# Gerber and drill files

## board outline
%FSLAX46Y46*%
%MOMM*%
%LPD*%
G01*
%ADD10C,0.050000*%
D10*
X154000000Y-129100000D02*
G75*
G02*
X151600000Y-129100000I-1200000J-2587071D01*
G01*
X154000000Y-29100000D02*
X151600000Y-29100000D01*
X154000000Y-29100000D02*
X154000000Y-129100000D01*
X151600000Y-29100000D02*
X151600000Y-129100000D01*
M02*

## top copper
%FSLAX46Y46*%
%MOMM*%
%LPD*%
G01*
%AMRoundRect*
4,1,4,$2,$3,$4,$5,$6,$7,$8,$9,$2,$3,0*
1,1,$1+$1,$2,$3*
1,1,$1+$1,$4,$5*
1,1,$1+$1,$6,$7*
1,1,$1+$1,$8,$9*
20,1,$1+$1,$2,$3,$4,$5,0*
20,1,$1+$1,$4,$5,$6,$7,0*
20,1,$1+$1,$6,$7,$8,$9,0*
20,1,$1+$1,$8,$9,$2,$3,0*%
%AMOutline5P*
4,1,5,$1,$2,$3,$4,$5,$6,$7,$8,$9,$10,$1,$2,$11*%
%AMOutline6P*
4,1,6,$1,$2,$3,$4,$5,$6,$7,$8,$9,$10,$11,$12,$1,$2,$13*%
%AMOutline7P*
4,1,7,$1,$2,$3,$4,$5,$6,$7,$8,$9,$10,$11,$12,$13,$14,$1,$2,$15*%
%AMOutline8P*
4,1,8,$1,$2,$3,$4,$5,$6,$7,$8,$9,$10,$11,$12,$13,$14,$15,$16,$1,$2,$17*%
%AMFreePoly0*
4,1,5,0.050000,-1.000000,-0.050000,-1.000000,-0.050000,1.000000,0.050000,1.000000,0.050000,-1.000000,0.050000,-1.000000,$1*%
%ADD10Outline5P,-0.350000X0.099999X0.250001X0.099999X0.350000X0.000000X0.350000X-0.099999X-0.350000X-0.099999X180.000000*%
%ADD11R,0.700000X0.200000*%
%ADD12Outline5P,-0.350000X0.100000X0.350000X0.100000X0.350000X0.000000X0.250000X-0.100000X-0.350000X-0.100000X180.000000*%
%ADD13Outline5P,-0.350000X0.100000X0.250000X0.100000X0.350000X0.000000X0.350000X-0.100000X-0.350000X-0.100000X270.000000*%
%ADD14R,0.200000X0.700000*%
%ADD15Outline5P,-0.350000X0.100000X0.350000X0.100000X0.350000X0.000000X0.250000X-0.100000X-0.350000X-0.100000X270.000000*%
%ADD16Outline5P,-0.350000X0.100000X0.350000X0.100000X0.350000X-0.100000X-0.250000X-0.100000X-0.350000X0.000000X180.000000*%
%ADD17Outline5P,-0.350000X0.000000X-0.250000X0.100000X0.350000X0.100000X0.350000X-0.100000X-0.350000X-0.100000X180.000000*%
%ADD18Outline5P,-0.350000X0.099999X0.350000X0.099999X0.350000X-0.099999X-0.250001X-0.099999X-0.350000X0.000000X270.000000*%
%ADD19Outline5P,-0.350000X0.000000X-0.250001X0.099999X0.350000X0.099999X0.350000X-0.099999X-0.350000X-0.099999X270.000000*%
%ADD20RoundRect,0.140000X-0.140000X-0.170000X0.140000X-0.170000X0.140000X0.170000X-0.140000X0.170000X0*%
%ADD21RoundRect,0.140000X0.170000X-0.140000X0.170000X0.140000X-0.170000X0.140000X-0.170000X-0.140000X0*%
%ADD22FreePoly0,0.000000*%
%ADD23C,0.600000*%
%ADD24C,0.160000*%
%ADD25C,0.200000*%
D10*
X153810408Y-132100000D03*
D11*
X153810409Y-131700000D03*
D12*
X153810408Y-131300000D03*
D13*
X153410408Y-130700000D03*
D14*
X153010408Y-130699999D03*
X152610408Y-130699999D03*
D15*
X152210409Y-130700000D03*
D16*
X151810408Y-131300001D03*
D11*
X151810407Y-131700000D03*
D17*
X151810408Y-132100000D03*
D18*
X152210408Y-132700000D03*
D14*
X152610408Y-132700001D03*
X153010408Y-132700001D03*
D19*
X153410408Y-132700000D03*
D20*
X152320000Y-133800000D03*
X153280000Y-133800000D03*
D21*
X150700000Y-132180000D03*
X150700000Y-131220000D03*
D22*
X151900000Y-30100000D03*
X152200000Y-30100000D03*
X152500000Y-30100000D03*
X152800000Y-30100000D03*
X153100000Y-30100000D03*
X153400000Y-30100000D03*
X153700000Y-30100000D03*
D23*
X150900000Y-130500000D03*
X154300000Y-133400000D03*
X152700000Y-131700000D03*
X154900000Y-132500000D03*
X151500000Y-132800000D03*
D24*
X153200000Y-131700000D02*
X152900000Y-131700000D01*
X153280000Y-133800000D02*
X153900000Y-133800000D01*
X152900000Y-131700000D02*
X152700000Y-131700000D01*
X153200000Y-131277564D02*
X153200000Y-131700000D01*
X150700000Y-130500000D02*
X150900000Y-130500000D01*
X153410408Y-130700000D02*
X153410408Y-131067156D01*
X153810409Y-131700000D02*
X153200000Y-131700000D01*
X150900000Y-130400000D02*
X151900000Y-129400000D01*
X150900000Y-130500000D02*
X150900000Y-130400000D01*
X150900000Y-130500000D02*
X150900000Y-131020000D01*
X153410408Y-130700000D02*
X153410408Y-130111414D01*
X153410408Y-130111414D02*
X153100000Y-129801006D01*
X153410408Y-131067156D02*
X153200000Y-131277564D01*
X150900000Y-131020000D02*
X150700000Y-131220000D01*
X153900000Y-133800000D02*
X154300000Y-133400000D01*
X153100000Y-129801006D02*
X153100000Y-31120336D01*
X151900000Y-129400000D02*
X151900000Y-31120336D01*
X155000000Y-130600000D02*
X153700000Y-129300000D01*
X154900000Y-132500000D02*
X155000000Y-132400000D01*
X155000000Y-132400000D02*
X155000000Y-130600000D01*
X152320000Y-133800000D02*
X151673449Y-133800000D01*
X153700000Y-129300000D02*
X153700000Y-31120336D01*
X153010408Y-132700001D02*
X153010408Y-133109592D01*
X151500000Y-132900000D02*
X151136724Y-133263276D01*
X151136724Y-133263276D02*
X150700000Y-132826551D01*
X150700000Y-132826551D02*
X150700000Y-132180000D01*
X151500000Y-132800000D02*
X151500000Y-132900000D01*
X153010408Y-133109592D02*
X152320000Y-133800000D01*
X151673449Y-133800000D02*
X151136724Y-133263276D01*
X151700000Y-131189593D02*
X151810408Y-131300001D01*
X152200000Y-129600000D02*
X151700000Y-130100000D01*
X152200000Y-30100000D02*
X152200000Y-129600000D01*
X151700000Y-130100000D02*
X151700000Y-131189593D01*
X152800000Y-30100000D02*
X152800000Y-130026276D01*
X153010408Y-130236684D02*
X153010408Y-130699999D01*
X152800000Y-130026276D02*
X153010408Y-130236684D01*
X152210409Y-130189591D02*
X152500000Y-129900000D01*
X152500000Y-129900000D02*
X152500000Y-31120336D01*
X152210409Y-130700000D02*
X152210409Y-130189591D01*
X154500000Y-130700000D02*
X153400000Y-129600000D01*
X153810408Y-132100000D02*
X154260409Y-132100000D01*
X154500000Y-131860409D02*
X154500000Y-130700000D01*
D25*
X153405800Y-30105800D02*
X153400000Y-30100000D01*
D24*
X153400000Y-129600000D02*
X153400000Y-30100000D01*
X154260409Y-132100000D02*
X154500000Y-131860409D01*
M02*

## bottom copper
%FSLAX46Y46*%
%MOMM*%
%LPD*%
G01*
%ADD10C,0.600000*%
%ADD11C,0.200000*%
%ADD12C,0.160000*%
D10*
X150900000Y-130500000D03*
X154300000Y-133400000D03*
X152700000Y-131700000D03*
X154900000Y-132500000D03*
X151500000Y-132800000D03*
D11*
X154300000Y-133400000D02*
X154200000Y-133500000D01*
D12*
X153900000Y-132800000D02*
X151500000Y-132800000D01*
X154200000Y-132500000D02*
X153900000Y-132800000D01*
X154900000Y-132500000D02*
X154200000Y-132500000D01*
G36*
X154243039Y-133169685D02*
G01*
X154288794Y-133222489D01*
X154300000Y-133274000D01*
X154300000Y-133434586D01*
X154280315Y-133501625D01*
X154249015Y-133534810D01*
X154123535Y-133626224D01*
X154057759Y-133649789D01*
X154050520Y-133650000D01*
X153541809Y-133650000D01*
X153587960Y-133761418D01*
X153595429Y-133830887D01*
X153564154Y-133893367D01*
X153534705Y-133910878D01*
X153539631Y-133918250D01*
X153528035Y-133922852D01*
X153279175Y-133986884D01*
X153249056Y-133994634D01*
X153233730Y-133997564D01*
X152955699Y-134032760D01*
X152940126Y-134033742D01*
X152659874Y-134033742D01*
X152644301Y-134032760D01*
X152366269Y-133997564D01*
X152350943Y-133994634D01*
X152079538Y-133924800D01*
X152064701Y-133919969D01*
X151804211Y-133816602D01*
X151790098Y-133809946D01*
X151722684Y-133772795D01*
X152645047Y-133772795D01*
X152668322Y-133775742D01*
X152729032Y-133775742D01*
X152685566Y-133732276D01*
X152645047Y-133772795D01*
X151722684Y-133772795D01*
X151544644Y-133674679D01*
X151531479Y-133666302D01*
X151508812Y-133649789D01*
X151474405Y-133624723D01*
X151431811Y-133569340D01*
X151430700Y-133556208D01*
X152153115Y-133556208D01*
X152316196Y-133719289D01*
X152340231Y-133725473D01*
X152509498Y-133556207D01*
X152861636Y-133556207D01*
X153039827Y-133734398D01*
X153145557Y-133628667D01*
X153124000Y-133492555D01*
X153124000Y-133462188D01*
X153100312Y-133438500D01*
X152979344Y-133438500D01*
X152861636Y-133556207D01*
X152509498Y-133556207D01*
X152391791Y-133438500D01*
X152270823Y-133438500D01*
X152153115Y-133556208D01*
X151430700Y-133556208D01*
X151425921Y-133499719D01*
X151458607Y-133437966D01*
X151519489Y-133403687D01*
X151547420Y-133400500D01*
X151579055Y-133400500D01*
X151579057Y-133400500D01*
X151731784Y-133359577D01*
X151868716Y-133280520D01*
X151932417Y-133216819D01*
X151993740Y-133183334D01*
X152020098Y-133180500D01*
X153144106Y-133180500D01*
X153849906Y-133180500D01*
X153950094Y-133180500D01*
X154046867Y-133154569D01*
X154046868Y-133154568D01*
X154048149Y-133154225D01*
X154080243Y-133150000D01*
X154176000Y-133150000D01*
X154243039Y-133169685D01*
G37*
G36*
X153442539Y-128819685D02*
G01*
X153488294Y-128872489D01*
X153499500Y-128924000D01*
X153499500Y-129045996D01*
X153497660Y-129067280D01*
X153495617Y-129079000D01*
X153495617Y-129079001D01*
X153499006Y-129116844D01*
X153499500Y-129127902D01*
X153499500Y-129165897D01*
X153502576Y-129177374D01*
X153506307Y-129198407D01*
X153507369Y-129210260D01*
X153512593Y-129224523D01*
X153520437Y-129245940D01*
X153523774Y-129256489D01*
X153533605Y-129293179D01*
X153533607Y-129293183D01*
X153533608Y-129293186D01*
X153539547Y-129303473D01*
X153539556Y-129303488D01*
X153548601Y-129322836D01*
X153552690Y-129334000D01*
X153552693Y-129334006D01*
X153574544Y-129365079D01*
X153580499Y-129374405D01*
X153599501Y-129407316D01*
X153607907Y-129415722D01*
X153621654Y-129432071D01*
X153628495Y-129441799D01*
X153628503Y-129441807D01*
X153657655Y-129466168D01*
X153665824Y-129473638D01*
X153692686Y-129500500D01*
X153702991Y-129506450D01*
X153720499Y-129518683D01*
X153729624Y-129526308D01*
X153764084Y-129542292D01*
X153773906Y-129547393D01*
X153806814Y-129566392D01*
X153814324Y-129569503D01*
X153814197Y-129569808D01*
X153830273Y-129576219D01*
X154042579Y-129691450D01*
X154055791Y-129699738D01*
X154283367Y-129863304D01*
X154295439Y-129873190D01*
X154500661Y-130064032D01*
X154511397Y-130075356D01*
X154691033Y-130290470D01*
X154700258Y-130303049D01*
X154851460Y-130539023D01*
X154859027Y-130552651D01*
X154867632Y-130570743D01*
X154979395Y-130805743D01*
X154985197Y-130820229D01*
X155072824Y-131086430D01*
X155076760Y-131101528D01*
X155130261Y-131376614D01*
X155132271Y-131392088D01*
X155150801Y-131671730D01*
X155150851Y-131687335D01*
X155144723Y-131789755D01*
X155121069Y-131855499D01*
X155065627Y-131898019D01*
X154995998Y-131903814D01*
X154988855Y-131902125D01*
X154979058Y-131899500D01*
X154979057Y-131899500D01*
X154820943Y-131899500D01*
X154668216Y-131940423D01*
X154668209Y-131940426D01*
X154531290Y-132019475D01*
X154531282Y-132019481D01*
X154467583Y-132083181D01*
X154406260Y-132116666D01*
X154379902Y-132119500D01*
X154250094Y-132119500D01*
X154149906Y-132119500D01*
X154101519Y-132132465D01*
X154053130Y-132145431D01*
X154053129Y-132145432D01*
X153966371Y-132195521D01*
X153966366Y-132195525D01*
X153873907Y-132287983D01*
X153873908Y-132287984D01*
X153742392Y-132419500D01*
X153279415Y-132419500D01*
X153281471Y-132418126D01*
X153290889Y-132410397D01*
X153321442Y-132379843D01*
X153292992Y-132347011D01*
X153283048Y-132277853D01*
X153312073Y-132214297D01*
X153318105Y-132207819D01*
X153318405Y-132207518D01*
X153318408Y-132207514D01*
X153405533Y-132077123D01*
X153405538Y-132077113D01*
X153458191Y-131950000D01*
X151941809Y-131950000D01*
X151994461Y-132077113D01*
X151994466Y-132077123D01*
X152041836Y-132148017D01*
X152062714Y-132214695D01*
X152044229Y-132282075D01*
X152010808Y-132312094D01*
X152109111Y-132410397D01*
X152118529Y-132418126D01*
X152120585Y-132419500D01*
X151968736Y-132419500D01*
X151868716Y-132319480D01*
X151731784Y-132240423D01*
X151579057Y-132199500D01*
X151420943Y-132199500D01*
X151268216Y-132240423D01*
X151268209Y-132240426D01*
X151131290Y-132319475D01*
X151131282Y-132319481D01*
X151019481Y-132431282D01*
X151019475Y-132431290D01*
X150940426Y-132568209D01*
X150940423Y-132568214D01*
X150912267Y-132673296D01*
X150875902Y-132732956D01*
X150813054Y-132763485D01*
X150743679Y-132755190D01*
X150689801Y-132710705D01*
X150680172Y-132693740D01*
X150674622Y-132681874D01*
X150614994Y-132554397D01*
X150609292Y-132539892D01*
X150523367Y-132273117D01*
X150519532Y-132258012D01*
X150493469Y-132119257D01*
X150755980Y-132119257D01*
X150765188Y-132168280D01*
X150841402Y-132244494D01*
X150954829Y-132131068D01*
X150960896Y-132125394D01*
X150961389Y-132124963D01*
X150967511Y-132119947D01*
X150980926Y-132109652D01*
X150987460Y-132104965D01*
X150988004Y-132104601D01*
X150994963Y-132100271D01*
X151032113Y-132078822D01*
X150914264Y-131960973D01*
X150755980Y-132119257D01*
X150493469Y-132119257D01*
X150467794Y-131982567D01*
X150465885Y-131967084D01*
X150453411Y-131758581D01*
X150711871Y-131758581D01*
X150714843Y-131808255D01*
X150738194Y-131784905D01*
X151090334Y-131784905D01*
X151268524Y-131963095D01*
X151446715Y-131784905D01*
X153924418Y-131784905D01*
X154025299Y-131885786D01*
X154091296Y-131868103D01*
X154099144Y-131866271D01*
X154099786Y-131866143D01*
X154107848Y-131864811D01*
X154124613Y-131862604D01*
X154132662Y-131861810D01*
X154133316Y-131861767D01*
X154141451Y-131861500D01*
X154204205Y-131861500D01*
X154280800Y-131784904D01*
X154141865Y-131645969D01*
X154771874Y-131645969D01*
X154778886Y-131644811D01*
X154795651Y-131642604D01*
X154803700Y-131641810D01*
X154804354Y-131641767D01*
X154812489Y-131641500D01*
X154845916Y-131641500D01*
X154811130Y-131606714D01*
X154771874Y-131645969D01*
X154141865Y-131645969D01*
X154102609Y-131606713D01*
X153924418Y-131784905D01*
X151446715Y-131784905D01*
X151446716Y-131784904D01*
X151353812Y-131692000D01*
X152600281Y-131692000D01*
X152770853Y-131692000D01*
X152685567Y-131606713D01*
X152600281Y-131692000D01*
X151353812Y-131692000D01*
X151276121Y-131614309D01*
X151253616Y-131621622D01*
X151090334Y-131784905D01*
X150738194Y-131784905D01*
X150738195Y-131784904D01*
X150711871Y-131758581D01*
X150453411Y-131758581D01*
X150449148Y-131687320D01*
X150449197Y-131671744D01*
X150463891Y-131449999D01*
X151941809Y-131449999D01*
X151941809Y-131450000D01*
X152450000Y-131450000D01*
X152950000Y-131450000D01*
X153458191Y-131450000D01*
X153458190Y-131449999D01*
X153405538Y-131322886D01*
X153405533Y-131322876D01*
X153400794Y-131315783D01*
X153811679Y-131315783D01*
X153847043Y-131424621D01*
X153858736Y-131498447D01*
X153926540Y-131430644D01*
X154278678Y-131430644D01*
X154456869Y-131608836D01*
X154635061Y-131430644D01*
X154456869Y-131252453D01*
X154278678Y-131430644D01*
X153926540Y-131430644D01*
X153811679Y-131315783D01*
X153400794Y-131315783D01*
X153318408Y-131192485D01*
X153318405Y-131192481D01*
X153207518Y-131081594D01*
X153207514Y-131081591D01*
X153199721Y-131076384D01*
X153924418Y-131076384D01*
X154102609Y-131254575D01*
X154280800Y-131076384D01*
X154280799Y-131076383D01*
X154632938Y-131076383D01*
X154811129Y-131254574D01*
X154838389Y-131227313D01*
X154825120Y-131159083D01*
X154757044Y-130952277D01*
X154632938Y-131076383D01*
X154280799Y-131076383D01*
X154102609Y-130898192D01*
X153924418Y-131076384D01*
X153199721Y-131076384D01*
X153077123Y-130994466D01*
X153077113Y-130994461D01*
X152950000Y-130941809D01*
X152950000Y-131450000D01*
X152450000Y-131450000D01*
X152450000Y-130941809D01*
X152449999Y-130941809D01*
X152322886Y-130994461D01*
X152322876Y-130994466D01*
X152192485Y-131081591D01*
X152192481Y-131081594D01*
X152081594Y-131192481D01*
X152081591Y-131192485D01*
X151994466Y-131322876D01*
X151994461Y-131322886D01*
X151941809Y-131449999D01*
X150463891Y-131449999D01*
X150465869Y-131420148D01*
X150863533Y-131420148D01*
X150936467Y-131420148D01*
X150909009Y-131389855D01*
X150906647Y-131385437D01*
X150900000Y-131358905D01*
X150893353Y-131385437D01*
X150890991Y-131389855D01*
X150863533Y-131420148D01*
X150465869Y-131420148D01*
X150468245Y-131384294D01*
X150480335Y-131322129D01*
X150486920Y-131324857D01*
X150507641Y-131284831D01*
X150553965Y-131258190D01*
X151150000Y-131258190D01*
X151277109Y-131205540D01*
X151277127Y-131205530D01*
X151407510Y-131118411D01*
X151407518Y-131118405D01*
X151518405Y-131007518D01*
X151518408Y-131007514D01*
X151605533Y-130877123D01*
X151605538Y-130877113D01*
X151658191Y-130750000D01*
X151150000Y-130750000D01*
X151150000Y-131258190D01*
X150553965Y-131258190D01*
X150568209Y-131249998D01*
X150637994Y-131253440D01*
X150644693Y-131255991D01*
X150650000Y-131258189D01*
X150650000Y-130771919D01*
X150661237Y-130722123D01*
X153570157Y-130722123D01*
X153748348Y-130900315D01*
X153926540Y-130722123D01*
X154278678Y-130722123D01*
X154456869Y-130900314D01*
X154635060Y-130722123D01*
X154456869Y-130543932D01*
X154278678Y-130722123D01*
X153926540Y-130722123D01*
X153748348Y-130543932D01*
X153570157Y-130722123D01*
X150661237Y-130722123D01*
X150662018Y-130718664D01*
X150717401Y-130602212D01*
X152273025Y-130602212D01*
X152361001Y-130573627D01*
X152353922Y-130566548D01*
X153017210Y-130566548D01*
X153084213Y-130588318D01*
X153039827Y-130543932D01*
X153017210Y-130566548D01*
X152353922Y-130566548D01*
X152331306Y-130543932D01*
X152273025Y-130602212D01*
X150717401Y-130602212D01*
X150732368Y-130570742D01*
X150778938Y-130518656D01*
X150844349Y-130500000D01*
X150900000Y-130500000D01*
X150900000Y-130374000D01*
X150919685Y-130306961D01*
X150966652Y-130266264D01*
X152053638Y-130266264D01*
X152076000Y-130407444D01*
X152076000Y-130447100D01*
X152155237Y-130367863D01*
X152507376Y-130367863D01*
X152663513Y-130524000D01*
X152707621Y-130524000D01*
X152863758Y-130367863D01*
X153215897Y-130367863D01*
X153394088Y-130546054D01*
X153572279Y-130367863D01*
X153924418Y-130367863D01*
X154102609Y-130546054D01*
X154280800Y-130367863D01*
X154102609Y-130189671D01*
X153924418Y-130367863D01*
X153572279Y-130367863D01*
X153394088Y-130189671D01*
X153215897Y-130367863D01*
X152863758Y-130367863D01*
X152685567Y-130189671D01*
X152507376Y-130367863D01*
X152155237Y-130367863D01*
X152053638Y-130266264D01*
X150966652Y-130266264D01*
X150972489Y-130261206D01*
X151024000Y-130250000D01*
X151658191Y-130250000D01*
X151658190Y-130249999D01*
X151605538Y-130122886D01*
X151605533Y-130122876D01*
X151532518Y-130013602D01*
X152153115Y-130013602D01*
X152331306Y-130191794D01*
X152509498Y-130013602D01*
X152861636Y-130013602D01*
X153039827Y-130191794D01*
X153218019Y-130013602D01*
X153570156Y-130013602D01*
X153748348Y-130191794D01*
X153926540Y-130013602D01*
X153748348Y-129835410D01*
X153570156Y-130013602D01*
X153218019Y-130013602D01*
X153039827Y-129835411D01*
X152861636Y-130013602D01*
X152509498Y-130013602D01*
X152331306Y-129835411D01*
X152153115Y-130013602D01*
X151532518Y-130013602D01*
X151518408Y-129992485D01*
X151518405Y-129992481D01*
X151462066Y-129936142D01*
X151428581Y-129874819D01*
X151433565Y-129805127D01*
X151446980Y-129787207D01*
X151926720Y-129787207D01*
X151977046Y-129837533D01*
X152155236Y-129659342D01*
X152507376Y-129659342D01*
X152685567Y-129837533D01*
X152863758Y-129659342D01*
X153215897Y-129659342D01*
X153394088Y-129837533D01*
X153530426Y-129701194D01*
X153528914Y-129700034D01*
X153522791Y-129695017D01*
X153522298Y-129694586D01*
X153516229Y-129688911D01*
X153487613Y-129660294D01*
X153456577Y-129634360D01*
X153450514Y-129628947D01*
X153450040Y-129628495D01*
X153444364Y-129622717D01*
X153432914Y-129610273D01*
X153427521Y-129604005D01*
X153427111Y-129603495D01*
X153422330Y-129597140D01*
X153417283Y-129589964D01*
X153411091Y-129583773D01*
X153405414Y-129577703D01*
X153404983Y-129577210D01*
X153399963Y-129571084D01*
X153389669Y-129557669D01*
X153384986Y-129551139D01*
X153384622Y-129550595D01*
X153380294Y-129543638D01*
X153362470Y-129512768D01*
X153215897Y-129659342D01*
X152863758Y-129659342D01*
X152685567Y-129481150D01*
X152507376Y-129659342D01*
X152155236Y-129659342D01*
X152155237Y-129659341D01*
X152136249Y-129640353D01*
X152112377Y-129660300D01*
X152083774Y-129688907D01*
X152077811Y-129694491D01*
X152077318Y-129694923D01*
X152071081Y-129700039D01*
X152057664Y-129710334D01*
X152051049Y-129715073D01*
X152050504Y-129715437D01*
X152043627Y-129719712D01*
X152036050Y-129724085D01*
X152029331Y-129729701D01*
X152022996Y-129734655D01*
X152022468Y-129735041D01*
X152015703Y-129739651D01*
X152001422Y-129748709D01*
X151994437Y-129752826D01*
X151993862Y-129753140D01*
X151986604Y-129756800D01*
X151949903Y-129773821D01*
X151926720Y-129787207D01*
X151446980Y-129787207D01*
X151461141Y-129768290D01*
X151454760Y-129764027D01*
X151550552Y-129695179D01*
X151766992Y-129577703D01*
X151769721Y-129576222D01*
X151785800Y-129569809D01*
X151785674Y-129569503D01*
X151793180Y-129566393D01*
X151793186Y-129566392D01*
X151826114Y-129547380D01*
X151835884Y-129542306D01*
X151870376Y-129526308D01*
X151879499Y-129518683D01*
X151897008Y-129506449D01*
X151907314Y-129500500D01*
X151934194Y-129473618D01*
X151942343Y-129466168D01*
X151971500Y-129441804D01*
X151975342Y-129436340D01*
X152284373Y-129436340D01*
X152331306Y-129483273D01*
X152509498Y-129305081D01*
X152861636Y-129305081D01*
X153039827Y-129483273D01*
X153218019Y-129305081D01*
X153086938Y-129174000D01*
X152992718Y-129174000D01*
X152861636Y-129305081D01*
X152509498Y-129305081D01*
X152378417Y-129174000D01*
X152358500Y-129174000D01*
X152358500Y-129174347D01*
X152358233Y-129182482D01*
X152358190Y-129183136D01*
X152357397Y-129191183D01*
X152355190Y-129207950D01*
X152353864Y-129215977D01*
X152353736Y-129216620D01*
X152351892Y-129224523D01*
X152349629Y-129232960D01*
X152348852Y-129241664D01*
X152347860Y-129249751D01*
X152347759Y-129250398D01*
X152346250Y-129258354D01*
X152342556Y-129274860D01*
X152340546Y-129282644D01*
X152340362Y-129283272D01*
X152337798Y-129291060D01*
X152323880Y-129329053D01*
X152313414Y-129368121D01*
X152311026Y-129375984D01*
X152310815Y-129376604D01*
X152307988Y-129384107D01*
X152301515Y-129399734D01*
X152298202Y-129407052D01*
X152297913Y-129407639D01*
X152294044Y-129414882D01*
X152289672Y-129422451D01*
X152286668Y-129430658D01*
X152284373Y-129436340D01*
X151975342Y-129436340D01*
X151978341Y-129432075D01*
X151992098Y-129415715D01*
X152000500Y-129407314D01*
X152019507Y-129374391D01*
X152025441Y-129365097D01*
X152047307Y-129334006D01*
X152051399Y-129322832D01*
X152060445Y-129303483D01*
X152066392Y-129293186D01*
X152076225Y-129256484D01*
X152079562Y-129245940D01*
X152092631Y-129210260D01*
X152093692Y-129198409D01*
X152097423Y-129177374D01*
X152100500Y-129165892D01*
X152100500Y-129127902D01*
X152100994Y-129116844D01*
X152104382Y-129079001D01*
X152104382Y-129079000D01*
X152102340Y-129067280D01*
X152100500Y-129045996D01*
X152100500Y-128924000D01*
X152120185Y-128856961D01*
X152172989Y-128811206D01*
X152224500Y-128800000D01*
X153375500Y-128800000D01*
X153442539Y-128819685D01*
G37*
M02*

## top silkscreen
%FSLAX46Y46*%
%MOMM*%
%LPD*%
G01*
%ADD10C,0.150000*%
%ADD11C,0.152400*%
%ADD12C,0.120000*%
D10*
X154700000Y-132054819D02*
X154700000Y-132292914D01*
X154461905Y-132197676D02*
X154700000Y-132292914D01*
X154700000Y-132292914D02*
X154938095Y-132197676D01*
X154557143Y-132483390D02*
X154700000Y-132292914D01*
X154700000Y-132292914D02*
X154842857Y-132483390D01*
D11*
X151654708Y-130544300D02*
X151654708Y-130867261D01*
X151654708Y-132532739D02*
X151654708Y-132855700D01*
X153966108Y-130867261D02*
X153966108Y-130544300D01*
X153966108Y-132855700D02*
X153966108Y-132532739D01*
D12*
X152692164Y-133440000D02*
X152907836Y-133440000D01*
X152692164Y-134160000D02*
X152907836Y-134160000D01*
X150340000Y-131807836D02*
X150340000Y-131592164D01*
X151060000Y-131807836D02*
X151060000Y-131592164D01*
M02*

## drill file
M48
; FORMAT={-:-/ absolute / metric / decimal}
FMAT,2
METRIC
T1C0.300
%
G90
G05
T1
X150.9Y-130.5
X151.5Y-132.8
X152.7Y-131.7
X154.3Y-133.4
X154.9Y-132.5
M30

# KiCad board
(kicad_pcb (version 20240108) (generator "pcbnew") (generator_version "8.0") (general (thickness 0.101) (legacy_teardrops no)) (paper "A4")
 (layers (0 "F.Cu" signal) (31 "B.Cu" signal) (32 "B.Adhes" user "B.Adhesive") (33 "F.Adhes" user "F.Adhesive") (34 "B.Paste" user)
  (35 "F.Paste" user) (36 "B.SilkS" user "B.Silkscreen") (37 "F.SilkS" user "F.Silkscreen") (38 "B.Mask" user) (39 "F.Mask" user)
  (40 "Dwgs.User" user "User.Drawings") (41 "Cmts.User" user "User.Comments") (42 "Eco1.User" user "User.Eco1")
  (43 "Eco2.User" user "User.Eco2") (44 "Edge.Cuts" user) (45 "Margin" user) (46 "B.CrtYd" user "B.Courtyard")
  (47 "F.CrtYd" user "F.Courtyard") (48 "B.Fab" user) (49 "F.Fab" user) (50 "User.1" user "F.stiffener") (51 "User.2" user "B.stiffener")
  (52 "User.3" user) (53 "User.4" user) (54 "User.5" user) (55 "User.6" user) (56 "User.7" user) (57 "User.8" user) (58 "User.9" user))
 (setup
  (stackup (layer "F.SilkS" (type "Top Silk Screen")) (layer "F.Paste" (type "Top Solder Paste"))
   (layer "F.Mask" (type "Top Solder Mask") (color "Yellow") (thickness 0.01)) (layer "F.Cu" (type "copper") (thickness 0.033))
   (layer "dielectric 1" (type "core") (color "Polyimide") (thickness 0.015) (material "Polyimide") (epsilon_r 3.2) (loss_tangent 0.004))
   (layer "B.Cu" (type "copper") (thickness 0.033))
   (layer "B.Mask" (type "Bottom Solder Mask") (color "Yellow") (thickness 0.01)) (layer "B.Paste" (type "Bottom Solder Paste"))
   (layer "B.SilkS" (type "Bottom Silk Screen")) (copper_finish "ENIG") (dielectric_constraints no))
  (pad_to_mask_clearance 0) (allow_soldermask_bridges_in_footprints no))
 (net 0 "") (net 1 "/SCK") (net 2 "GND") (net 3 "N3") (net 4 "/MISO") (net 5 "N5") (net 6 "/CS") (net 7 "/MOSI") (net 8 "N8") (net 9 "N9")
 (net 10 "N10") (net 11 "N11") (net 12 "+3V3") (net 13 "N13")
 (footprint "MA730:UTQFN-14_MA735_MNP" (layer "F.Cu") (at 152.810408 131.7 180)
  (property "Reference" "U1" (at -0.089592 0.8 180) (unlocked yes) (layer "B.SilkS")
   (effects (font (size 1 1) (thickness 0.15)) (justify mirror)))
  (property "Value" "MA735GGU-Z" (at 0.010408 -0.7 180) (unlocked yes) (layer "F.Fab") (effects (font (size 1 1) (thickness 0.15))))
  (fp_line (start 1.1557 1.1557) (end 1.1557 0.832739) (stroke (width 0.1524) (type solid)) (layer "F.SilkS"))
  (fp_line (start 1.1557 -0.832739) (end 1.1557 -1.1557) (stroke (width 0.1524) (type solid)) (layer "F.SilkS"))
  (fp_line (start -1.1557 0.832739) (end -1.1557 1.1557) (stroke (width 0.1524) (type solid)) (layer "F.SilkS"))
  (fp_line (start -1.1557 -1.1557) (end -1.1557 -0.832739) (stroke (width 0.1524) (type solid)) (layer "F.SilkS"))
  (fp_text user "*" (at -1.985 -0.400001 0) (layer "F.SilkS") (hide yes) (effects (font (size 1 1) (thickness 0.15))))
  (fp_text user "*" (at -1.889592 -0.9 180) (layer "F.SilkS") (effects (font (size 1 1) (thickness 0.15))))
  (pad "1" smd roundrect (at -1 -0.4 180) (size 0.7 0.199998) (layers "F.Cu" "F.Paste" "F.Mask") (roundrect_rratio 0) (chamfer_ratio 0.5)
   (chamfer top_right) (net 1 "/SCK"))
  (pad "2" smd rect (at -1.000001 0 180) (size 0.7 0.2) (layers "F.Cu" "F.Paste" "F.Mask") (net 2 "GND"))
  (pad "3" smd roundrect (at -1 0.4 180) (size 0.7 0.2) (layers "F.Cu" "F.Paste" "F.Mask") (roundrect_rratio 0) (chamfer_ratio 0.5)
   (chamfer bottom_right) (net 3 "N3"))
  (pad "4" smd roundrect (at -0.6 1 270) (size 0.7 0.2) (layers "F.Cu" "F.Paste" "F.Mask") (roundrect_rratio 0) (chamfer_ratio 0.5)
   (chamfer top_right) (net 2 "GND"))
  (pad "5" smd rect (at -0.2 1.000001 270) (size 0.7 0.2) (layers "F.Cu" "F.Paste" "F.Mask") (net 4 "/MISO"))
  (pad "6" smd rect (at 0.2 1.000001 270) (size 0.7 0.2) (layers "F.Cu" "F.Paste" "F.Mask") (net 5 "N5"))
  (pad "7" smd roundrect (at 0.599999 1 270) (size 0.7 0.199999) (layers "F.Cu" "F.Paste" "F.Mask") (roundrect_rratio 0) (chamfer_ratio 0.5)
   (chamfer bottom_right) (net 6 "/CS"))
  (pad "8" smd roundrect (at 1 0.399999 180) (size 0.7 0.2) (layers "F.Cu" "F.Paste" "F.Mask") (roundrect_rratio 0) (chamfer_ratio 0.5)
   (chamfer bottom_left) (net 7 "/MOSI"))
  (pad "9" smd rect (at 1.000001 0 180) (size 0.7 0.2) (layers "F.Cu" "F.Paste" "F.Mask") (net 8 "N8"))
  (pad "10" smd roundrect (at 1 -0.4 180) (size 0.7 0.2) (layers "F.Cu" "F.Paste" "F.Mask") (roundrect_rratio 0) (chamfer_ratio 0.5)
   (chamfer top_left) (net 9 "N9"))
  (pad "11" smd roundrect (at 0.6 -1 270) (size 0.7 0.199998) (layers "F.Cu" "F.Paste" "F.Mask") (roundrect_rratio 0) (chamfer_ratio 0.5)
   (chamfer bottom_left) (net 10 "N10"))
  (pad "12" smd rect (at 0.2 -1.000001 270) (size 0.7 0.2) (layers "F.Cu" "F.Paste" "F.Mask") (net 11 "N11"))
  (pad "13" smd rect (at -0.2 -1.000001 270) (size 0.7 0.2) (layers "F.Cu" "F.Paste" "F.Mask") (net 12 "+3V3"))
  (pad "14" smd roundrect (at -0.6 -1 270) (size 0.7 0.199998) (layers "F.Cu" "F.Paste" "F.Mask") (roundrect_rratio 0) (chamfer_ratio 0.5)
   (chamfer top_left) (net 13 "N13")))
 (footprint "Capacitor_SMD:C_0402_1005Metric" (layer "F.Cu") (at 152.8 133.8)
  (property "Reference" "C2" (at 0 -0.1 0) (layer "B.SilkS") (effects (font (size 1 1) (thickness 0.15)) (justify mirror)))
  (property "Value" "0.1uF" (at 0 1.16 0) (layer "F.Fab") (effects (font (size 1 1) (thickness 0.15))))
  (fp_line (start -0.107836 -0.36) (end 0.107836 -0.36) (stroke (width 0.12) (type solid)) (layer "F.SilkS"))
  (fp_line (start -0.107836 0.36) (end 0.107836 0.36) (stroke (width 0.12) (type solid)) (layer "F.SilkS"))
  (pad "1" smd roundrect (at -0.48 0) (size 0.56 0.62) (layers "F.Cu" "F.Paste" "F.Mask") (roundrect_rratio 0.25) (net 12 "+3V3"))
  (pad "2" smd roundrect (at 0.48 0) (size 0.56 0.62) (layers "F.Cu" "F.Paste" "F.Mask") (roundrect_rratio 0.25) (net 2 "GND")))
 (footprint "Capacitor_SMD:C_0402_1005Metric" (layer "F.Cu") (at 150.7 131.7 90)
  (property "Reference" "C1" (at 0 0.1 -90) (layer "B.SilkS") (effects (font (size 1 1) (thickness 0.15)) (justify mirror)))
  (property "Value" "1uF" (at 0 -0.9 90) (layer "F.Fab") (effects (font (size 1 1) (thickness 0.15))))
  (fp_line (start -0.107836 -0.36) (end 0.107836 -0.36) (stroke (width 0.12) (type solid)) (layer "F.SilkS"))
  (fp_line (start -0.107836 0.36) (end 0.107836 0.36) (stroke (width 0.12) (type solid)) (layer "F.SilkS"))
  (pad "1" smd roundrect (at -0.48 0 90) (size 0.56 0.62) (layers "F.Cu" "F.Paste" "F.Mask") (roundrect_rratio 0.25) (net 12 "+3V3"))
  (pad "2" smd roundrect (at 0.48 0 90) (size 0.56 0.62) (layers "F.Cu" "F.Paste" "F.Mask") (roundrect_rratio 0.25) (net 2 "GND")))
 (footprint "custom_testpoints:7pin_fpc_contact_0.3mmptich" (layer "F.Cu") (at 152.8 30.2)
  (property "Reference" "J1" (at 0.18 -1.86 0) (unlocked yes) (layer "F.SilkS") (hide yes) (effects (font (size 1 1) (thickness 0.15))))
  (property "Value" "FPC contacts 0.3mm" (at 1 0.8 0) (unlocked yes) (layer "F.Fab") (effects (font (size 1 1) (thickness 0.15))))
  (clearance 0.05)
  (pad "1" connect custom (at -0.9 -0.1) (size 0.1 2) (layers "F.Cu" "F.Mask") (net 2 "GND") (clearance 0.05)
   (options (clearance outline) (anchor rect)) (primitives))
  (pad "2" connect custom (at -0.6 -0.1) (size 0.1 2) (layers "F.Cu" "F.Mask") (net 7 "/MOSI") (clearance 0.05)
   (options (clearance outline) (anchor rect)) (primitives))
  (pad "3" connect custom (at -0.3 -0.1) (size 0.1 2) (layers "F.Cu" "F.Mask") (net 6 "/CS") (clearance 0.05)
   (options (clearance outline) (anchor rect)) (primitives))
  (pad "4" connect custom (at 0 -0.1) (size 0.1 2) (layers "F.Cu" "F.Mask") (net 4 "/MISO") (clearance 0.05)
   (options (clearance outline) (anchor rect)) (primitives))
  (pad "5" connect custom (at 0.3 -0.1) (size 0.1 2) (layers "F.Cu" "F.Mask") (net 2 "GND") (clearance 0.05)
   (options (clearance outline) (anchor rect)) (primitives))
  (pad "6" connect custom (at 0.6 -0.1) (size 0.1 2) (layers "F.Cu" "F.Mask") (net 1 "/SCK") (clearance 0.05)
   (options (clearance outline) (anchor rect)) (primitives))
  (pad "7" connect custom (at 0.9 -0.1) (size 0.1 2) (layers "F.Cu" "F.Mask") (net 12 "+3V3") (clearance 0.05)
   (options (clearance outline) (anchor rect)) (primitives)))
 (gr_arc (start 154 129.1) (mid 152.8 134.538901) (end 151.6 129.1) (stroke (width 0.05) (type default)) (layer "Edge.Cuts"))
 (gr_line (start 154 29.1) (end 151.6 29.1) (stroke (width 0.05) (type default)) (layer "Edge.Cuts"))
 (gr_line (start 154 29.1) (end 154 129.1) (stroke (width 0.05) (type default)) (layer "Edge.Cuts"))
 (gr_line (start 151.6 29.1) (end 151.6 129.1) (stroke (width 0.05) (type default)) (layer "Edge.Cuts"))
 (segment (start 153.2 131.7) (end 152.9 131.7) (width 0.16) (layer "F.Cu") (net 2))
 (segment (start 153.28 133.8) (end 153.9 133.8) (width 0.16) (layer "F.Cu") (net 2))
 (segment (start 152.9 131.7) (end 152.7 131.7) (width 0.16) (layer "F.Cu") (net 2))
 (segment (start 153.2 131.277564) (end 153.2 131.7) (width 0.16) (layer "F.Cu") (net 2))
 (segment (start 150.7 130.5) (end 150.9 130.5) (width 0.16) (layer "F.Cu") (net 2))
 (segment (start 153.410408 130.7) (end 153.410408 131.067156) (width 0.16) (layer "F.Cu") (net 2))
 (segment (start 153.810409 131.7) (end 153.2 131.7) (width 0.16) (layer "F.Cu") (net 2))
 (segment (start 150.9 130.4) (end 151.9 129.4) (width 0.16) (layer "F.Cu") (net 2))
 (segment (start 150.9 130.5) (end 150.9 130.4) (width 0.16) (layer "F.Cu") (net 2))
 (segment (start 150.9 130.5) (end 150.9 131.02) (width 0.16) (layer "F.Cu") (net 2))
 (segment (start 153.410408 130.7) (end 153.410408 130.111414) (width 0.16) (layer "F.Cu") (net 2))
 (segment (start 153.410408 130.111414) (end 153.1 129.801006) (width 0.16) (layer "F.Cu") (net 2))
 (segment (start 153.410408 131.067156) (end 153.2 131.277564) (width 0.16) (layer "F.Cu") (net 2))
 (segment (start 150.9 131.02) (end 150.7 131.22) (width 0.16) (layer "F.Cu") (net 2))
 (segment (start 153.9 133.8) (end 154.3 133.4) (width 0.16) (layer "F.Cu") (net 2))
 (segment (start 153.1 129.801006) (end 153.1 31.120336) (width 0.16) (layer "F.Cu") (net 2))
 (segment (start 151.9 129.4) (end 151.9 31.120336) (width 0.16) (layer "F.Cu") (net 2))
 (via (at 150.9 130.5) (size 0.6) (drill 0.3) (layers "F.Cu" "B.Cu") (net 2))
 (via (at 154.3 133.4) (size 0.6) (drill 0.3) (layers "F.Cu" "B.Cu") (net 2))
 (via (at 152.7 131.7) (size 0.6) (drill 0.3) (layers "F.Cu" "B.Cu") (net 2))
 (segment (start 154.3 133.4) (end 154.2 133.5) (width 0.2) (layer "B.Cu") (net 2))
 (segment (start 155 130.6) (end 153.7 129.3) (width 0.16) (layer "F.Cu") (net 12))
 (segment (start 154.9 132.5) (end 155 132.4) (width 0.16) (layer "F.Cu") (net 12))
 (segment (start 155 132.4) (end 155 130.6) (width 0.16) (layer "F.Cu") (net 12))
 (segment (start 152.32 133.8) (end 151.673449 133.8) (width 0.16) (layer "F.Cu") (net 12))
 (segment (start 153.7 129.3) (end 153.7 31.120336) (width 0.16) (layer "F.Cu") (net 12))
 (segment (start 153.010408 132.700001) (end 153.010408 133.109592) (width 0.16) (layer "F.Cu") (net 12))
 (segment (start 151.5 132.9) (end 151.136724 133.263276) (width 0.16) (layer "F.Cu") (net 12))
 (segment (start 151.136724 133.263276) (end 150.7 132.826551) (width 0.16) (layer "F.Cu") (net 12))
 (segment (start 150.7 132.826551) (end 150.7 132.18) (width 0.16) (layer "F.Cu") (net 12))
 (segment (start 151.5 132.8) (end 151.5 132.9) (width 0.16) (layer "F.Cu") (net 12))
 (segment (start 153.010408 133.109592) (end 152.32 133.8) (width 0.16) (layer "F.Cu") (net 12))
 (segment (start 151.673449 133.8) (end 151.136724 133.263276) (width 0.16) (layer "F.Cu") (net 12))
 (via (at 154.9 132.5) (size 0.6) (drill 0.3) (layers "F.Cu" "B.Cu") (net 12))
 (via (at 151.5 132.8) (size 0.6) (drill 0.3) (layers "F.Cu" "B.Cu") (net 12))
 (segment (start 153.9 132.8) (end 151.5 132.8) (width 0.16) (layer "B.Cu") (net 12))
 (segment (start 154.2 132.5) (end 153.9 132.8) (width 0.16) (layer "B.Cu") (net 12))
 (segment (start 154.9 132.5) (end 154.2 132.5) (width 0.16) (layer "B.Cu") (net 12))
 (segment (start 151.7 131.189593) (end 151.810408 131.300001) (width 0.16) (layer "F.Cu") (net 7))
 (segment (start 152.2 129.6) (end 151.7 130.1) (width 0.16) (layer "F.Cu") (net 7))
 (segment (start 152.2 30.1) (end 152.2 129.6) (width 0.16) (layer "F.Cu") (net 7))
 (segment (start 151.7 130.1) (end 151.7 131.189593) (width 0.16) (layer "F.Cu") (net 7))
 (segment (start 152.8 30.1) (end 152.8 130.026276) (width 0.16) (layer "F.Cu") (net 4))
 (segment (start 153.010408 130.236684) (end 153.010408 130.699999) (width 0.16) (layer "F.Cu") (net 4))
 (segment (start 152.8 130.026276) (end 153.010408 130.236684) (width 0.16) (layer "F.Cu") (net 4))
 (segment (start 152.210409 130.189591) (end 152.5 129.9) (width 0.16) (layer "F.Cu") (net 6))
 (segment (start 152.5 129.9) (end 152.5 31.120336) (width 0.16) (layer "F.Cu") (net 6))
 (segment (start 152.210409 130.7) (end 152.210409 130.189591) (width 0.16) (layer "F.Cu") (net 6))
 (segment (start 154.5 130.7) (end 153.4 129.6) (width 0.16) (layer "F.Cu") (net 1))
 (segment (start 153.810408 132.1) (end 154.260409 132.1) (width 0.16) (layer "F.Cu") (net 1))
 (segment (start 154.5 131.860409) (end 154.5 130.7) (width 0.16) (layer "F.Cu") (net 1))
 (segment (start 153.4058 30.1058) (end 153.4 30.1) (width 0.2) (layer "F.Cu") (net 1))
 (segment (start 153.4 129.6) (end 153.4 30.1) (width 0.16) (layer "F.Cu") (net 1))
 (segment (start 154.260409 132.1) (end 154.5 131.860409) (width 0.16) (layer "F.Cu") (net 1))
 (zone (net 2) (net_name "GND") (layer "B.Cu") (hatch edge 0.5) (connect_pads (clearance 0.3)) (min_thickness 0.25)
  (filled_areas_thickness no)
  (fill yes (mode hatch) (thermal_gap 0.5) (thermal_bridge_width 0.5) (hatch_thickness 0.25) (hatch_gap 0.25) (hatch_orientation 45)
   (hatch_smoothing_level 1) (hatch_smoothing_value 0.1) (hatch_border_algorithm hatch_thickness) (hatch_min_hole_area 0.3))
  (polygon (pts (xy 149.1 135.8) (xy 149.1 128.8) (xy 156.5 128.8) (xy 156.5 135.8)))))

